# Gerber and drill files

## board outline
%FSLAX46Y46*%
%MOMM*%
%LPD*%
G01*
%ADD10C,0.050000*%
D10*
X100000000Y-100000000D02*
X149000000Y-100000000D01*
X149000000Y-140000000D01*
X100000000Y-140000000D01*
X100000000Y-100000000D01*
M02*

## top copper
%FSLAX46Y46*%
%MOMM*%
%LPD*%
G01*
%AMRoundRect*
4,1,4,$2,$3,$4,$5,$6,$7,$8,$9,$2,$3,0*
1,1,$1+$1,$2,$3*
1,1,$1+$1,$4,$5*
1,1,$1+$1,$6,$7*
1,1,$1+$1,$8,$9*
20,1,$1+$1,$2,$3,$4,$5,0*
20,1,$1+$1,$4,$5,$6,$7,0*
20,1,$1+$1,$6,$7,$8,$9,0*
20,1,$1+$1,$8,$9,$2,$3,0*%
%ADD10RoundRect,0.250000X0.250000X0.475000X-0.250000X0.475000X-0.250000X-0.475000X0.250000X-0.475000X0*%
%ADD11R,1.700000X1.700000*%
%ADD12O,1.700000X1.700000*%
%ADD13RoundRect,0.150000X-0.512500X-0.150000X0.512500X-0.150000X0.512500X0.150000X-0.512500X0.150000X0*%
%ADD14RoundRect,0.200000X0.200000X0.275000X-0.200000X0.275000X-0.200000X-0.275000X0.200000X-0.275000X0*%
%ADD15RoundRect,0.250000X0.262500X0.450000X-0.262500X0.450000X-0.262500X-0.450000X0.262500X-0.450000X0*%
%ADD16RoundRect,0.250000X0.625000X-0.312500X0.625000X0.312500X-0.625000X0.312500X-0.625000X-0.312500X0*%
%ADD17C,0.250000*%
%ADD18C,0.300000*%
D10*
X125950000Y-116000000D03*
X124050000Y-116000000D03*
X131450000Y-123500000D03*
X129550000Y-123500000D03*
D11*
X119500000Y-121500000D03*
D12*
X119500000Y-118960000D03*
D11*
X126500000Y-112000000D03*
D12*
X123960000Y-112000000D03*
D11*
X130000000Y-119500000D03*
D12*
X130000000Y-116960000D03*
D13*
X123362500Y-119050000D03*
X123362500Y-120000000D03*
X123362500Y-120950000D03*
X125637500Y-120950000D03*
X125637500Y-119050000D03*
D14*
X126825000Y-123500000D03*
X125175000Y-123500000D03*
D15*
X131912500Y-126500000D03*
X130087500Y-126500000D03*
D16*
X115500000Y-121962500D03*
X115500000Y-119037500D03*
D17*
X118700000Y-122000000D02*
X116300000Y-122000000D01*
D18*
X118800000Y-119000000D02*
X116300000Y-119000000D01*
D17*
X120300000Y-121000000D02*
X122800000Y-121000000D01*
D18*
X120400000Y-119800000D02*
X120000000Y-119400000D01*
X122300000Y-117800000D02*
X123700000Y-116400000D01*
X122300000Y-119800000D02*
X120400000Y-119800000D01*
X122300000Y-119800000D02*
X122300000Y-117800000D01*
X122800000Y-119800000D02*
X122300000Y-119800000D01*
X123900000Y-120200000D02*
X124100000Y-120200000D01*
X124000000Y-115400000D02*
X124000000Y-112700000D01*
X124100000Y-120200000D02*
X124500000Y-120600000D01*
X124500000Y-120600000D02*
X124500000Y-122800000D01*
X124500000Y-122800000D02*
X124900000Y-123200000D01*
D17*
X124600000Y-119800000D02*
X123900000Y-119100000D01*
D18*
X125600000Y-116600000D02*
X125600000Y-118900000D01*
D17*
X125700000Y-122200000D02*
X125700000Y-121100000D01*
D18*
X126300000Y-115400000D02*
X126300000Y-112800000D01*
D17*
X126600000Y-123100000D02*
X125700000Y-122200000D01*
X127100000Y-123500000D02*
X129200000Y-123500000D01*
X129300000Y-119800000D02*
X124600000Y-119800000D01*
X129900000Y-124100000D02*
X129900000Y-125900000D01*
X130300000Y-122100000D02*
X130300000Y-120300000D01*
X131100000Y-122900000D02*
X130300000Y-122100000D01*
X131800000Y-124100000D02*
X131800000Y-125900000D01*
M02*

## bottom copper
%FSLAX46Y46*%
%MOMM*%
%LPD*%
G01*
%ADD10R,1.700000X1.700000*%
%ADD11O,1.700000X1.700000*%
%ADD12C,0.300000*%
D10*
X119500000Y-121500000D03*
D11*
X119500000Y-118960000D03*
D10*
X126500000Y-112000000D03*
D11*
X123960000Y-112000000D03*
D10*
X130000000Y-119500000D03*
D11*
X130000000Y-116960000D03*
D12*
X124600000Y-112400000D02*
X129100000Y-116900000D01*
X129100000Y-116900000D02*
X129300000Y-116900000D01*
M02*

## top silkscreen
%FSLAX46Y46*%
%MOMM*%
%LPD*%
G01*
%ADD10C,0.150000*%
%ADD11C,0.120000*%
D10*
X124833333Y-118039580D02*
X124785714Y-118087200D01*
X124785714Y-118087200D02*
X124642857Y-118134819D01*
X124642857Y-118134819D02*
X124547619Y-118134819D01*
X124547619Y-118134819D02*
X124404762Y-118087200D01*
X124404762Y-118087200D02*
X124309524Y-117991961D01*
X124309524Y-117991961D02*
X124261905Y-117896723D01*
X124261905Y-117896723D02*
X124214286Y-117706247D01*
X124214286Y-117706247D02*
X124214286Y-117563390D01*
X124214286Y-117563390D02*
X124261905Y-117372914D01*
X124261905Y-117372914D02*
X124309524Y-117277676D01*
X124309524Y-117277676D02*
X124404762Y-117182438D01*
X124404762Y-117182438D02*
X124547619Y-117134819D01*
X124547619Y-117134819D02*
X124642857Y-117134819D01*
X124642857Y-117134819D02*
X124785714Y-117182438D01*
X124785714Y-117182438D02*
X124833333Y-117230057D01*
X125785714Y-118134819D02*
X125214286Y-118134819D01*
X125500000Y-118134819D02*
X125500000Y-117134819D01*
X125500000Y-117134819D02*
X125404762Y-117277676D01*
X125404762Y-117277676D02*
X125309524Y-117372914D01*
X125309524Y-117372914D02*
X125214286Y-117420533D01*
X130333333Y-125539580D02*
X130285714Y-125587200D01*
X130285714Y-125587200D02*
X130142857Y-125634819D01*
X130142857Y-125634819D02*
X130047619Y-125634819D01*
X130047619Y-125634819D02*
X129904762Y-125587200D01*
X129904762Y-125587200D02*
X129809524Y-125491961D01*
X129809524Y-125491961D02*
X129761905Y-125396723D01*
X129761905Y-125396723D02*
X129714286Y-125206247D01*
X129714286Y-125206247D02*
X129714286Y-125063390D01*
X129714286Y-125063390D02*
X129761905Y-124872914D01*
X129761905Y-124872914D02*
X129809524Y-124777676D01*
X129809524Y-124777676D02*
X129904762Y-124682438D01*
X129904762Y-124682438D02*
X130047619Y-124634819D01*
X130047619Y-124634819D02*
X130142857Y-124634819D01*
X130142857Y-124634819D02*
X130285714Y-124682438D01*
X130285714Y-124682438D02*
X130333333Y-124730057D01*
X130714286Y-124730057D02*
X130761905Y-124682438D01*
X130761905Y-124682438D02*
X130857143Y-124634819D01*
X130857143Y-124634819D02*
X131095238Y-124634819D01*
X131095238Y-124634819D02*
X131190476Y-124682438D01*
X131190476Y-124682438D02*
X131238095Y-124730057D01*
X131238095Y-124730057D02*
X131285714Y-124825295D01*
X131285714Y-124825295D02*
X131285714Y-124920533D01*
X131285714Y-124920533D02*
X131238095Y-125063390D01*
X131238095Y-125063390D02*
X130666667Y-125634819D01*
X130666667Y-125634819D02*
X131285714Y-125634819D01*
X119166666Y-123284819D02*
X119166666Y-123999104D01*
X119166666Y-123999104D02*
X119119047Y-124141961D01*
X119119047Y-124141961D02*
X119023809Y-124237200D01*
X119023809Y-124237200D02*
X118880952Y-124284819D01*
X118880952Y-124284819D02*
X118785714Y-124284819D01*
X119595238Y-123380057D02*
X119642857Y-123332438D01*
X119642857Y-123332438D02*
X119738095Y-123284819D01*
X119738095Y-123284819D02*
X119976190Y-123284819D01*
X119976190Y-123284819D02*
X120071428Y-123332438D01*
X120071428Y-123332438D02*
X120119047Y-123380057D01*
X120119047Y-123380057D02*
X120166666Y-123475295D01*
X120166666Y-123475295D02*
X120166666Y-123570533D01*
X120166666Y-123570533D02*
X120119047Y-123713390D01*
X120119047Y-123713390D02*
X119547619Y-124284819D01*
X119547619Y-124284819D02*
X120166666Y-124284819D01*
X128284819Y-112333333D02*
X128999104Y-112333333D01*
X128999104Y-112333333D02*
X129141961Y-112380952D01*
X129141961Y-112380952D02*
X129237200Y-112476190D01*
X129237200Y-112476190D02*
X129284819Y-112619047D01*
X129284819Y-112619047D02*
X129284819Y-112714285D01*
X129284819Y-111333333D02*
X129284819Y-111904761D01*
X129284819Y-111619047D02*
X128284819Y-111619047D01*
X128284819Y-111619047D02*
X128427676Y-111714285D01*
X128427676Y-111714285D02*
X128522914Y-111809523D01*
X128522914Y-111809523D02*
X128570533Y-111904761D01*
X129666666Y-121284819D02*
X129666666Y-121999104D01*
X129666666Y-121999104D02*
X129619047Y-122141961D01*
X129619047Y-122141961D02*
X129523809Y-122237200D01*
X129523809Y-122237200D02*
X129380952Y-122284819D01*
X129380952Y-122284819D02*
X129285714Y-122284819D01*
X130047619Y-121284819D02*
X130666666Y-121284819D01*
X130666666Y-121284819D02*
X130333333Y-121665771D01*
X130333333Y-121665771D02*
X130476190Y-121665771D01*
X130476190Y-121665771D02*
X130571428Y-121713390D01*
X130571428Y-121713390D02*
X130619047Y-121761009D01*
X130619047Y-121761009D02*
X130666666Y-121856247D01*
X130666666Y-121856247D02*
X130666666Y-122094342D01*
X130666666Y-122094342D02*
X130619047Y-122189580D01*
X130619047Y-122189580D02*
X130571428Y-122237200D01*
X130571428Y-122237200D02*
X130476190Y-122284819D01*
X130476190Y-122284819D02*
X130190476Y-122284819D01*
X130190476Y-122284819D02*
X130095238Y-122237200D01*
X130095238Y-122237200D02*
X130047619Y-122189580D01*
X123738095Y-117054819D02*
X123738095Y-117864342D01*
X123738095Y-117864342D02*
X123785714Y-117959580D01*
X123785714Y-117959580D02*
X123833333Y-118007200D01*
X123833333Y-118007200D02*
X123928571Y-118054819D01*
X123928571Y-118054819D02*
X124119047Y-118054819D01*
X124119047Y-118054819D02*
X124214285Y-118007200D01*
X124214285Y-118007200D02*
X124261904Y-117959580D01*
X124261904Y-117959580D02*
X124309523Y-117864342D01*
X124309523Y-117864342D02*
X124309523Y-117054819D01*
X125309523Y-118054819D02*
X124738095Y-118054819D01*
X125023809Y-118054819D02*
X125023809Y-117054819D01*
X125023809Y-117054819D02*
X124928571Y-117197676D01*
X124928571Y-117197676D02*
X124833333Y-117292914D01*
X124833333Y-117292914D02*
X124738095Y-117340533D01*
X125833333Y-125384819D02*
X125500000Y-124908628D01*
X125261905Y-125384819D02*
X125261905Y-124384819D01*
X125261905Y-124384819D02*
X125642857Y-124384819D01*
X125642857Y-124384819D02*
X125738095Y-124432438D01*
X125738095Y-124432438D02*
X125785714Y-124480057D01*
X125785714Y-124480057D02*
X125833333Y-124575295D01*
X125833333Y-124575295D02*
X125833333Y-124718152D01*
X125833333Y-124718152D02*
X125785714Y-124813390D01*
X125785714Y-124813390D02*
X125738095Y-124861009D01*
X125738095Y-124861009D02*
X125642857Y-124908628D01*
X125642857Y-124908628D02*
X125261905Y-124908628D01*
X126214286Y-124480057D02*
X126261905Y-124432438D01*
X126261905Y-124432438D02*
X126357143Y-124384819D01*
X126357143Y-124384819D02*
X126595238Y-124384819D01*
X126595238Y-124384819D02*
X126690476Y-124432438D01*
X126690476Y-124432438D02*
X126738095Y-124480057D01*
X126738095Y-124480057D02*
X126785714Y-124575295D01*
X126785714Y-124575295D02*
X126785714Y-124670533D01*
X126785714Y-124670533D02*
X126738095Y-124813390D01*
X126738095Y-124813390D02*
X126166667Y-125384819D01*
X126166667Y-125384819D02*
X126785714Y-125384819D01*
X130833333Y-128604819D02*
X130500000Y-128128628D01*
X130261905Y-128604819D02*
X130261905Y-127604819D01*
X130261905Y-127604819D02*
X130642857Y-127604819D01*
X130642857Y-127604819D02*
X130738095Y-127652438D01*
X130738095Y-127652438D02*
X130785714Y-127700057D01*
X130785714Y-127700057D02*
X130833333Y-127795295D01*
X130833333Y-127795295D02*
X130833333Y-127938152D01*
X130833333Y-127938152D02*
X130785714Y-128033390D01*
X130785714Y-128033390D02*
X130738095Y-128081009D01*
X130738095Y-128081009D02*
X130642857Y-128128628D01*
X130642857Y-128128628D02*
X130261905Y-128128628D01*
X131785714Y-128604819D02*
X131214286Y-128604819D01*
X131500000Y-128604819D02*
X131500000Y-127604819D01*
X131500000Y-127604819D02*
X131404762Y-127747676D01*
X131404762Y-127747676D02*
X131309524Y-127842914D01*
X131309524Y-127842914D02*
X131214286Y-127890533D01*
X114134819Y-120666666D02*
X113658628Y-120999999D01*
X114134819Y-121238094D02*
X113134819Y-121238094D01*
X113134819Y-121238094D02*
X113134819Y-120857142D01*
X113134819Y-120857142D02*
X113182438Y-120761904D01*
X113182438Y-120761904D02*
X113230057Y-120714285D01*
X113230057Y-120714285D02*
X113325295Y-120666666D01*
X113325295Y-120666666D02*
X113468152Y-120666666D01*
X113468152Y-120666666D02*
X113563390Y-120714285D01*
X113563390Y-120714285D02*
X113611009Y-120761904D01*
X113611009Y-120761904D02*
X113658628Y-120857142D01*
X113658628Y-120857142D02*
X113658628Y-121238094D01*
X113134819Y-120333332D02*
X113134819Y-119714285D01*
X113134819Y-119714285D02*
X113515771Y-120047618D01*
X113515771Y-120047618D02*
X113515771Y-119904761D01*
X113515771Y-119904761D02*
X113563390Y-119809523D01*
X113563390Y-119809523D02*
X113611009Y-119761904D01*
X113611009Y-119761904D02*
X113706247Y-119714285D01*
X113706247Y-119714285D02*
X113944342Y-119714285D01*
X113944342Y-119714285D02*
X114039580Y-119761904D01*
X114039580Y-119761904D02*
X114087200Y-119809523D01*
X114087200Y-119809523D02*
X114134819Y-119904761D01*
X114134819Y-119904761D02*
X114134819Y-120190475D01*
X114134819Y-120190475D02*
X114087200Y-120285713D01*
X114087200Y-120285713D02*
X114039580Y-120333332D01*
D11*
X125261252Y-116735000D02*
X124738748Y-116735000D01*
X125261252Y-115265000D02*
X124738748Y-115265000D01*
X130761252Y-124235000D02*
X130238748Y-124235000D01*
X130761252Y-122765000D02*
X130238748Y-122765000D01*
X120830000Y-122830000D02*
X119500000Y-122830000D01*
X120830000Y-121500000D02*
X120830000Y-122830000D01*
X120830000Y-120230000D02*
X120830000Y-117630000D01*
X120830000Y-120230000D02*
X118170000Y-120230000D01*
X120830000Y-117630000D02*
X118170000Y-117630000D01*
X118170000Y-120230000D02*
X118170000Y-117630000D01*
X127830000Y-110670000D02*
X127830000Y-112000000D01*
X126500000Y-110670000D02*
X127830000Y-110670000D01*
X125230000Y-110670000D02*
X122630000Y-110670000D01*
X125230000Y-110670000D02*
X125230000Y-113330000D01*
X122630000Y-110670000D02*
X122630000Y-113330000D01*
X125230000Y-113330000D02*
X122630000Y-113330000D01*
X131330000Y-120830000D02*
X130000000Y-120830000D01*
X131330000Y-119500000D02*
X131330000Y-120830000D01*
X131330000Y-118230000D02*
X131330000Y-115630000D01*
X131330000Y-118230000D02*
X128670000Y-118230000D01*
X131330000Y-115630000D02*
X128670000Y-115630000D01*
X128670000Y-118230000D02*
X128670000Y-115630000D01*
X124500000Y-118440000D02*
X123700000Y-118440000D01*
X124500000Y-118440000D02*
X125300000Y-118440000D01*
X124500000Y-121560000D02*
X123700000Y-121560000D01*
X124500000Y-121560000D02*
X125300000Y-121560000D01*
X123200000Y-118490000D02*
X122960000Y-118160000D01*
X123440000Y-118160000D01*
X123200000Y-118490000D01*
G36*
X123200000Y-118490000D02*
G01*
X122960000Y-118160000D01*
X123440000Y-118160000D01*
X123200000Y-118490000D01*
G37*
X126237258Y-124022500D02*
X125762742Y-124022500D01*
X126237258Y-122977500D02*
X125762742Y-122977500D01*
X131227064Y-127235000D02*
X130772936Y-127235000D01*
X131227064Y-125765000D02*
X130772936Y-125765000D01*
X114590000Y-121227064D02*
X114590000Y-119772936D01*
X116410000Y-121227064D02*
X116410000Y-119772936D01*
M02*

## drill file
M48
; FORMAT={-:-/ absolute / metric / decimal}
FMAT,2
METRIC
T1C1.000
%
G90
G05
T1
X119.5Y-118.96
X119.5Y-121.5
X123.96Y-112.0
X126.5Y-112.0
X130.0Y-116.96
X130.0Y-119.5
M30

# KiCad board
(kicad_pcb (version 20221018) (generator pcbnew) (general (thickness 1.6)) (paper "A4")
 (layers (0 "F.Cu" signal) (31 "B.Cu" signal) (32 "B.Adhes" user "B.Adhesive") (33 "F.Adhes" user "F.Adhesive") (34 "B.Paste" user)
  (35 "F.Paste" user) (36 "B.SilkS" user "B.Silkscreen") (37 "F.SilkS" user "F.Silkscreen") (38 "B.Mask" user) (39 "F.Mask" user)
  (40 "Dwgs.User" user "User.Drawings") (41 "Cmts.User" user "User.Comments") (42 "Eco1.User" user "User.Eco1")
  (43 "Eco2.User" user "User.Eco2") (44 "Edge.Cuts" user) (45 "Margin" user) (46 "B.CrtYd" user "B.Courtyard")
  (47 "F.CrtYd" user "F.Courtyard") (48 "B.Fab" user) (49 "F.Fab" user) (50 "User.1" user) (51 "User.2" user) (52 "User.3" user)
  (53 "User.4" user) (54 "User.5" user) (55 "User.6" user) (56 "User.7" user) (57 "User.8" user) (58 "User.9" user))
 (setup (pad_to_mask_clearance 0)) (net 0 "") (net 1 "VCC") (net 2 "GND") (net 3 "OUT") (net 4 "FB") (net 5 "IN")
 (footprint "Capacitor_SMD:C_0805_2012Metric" (layer "F.Cu") (at 125 116 180)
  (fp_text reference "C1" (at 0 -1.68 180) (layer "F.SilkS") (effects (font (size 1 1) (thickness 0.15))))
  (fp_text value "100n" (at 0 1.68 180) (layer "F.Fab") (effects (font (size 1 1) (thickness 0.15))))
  (fp_line (start -0.261252 -0.735) (end 0.261252 -0.735) (stroke (width 0.12) (type solid)) (layer "F.SilkS"))
  (fp_line (start -0.261252 0.735) (end 0.261252 0.735) (stroke (width 0.12) (type solid)) (layer "F.SilkS"))
  (pad "1" smd roundrect (at -0.95 0 180) (size 1 1.45) (layers "F.Cu" "F.Paste" "F.Mask") (roundrect_rratio 0.25) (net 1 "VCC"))
  (pad "2" smd roundrect (at 0.95 0 180) (size 1 1.45) (layers "F.Cu" "F.Paste" "F.Mask") (roundrect_rratio 0.25) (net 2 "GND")))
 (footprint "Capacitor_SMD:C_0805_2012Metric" (layer "F.Cu") (at 130.5 123.5 180)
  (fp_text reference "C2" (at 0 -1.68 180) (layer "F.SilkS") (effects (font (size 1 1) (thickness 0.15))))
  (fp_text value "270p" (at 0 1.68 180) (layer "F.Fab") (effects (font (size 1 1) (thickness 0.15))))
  (fp_line (start -0.261252 -0.735) (end 0.261252 -0.735) (stroke (width 0.12) (type solid)) (layer "F.SilkS"))
  (fp_line (start -0.261252 0.735) (end 0.261252 0.735) (stroke (width 0.12) (type solid)) (layer "F.SilkS"))
  (pad "1" smd roundrect (at -0.95 0 180) (size 1 1.45) (layers "F.Cu" "F.Paste" "F.Mask") (roundrect_rratio 0.25) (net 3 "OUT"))
  (pad "2" smd roundrect (at 0.95 0 180) (size 1 1.45) (layers "F.Cu" "F.Paste" "F.Mask") (roundrect_rratio 0.25) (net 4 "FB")))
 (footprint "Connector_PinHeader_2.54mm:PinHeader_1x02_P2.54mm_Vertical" (layer "F.Cu") (at 119.5 121.5 180)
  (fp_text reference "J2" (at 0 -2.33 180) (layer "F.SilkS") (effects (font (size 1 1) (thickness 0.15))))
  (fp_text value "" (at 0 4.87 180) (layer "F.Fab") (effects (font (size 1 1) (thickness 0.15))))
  (fp_line (start -1.33 -1.33) (end 0 -1.33) (stroke (width 0.12) (type solid)) (layer "F.SilkS"))
  (fp_line (start -1.33 0) (end -1.33 -1.33) (stroke (width 0.12) (type solid)) (layer "F.SilkS"))
  (fp_line (start -1.33 1.27) (end -1.33 3.87) (stroke (width 0.12) (type solid)) (layer "F.SilkS"))
  (fp_line (start -1.33 1.27) (end 1.33 1.27) (stroke (width 0.12) (type solid)) (layer "F.SilkS"))
  (fp_line (start -1.33 3.87) (end 1.33 3.87) (stroke (width 0.12) (type solid)) (layer "F.SilkS"))
  (fp_line (start 1.33 1.27) (end 1.33 3.87) (stroke (width 0.12) (type solid)) (layer "F.SilkS"))
  (pad "1" thru_hole rect (at 0 0 180) (size 1.7 1.7) (drill 1) (layers "*.Cu" "*.Mask") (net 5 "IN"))
  (pad "2" thru_hole oval (at 0 2.54 180) (size 1.7 1.7) (drill 1) (layers "*.Cu" "*.Mask") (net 2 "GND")))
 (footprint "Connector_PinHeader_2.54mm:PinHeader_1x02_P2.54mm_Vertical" (layer "F.Cu") (at 126.5 112 -90)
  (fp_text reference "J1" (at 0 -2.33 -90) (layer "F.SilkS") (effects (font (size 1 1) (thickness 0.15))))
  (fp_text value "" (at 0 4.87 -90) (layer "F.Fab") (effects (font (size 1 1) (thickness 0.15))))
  (fp_line (start -1.33 -1.33) (end 0 -1.33) (stroke (width 0.12) (type solid)) (layer "F.SilkS"))
  (fp_line (start -1.33 0) (end -1.33 -1.33) (stroke (width 0.12) (type solid)) (layer "F.SilkS"))
  (fp_line (start -1.33 1.27) (end -1.33 3.87) (stroke (width 0.12) (type solid)) (layer "F.SilkS"))
  (fp_line (start -1.33 1.27) (end 1.33 1.27) (stroke (width 0.12) (type solid)) (layer "F.SilkS"))
  (fp_line (start -1.33 3.87) (end 1.33 3.87) (stroke (width 0.12) (type solid)) (layer "F.SilkS"))
  (fp_line (start 1.33 1.27) (end 1.33 3.87) (stroke (width 0.12) (type solid)) (layer "F.SilkS"))
  (pad "1" thru_hole rect (at 0 0 270) (size 1.7 1.7) (drill 1) (layers "*.Cu" "*.Mask") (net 1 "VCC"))
  (pad "2" thru_hole oval (at 0 2.54 270) (size 1.7 1.7) (drill 1) (layers "*.Cu" "*.Mask") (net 2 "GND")))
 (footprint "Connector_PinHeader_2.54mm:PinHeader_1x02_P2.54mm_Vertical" (layer "F.Cu") (at 130 119.5 180)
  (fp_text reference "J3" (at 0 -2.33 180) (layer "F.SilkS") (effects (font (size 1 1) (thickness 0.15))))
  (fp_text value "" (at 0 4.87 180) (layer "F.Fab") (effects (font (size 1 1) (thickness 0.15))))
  (fp_line (start -1.33 -1.33) (end 0 -1.33) (stroke (width 0.12) (type solid)) (layer "F.SilkS"))
  (fp_line (start -1.33 0) (end -1.33 -1.33) (stroke (width 0.12) (type solid)) (layer "F.SilkS"))
  (fp_line (start -1.33 1.27) (end -1.33 3.87) (stroke (width 0.12) (type solid)) (layer "F.SilkS"))
  (fp_line (start -1.33 1.27) (end 1.33 1.27) (stroke (width 0.12) (type solid)) (layer "F.SilkS"))
  (fp_line (start -1.33 3.87) (end 1.33 3.87) (stroke (width 0.12) (type solid)) (layer "F.SilkS"))
  (fp_line (start 1.33 1.27) (end 1.33 3.87) (stroke (width 0.12) (type solid)) (layer "F.SilkS"))
  (pad "1" thru_hole rect (at 0 0 180) (size 1.7 1.7) (drill 1) (layers "*.Cu" "*.Mask") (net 3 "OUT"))
  (pad "2" thru_hole oval (at 0 2.54 180) (size 1.7 1.7) (drill 1) (layers "*.Cu" "*.Mask") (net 2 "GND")))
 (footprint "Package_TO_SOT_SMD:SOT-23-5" (layer "F.Cu") (at 124.5 120)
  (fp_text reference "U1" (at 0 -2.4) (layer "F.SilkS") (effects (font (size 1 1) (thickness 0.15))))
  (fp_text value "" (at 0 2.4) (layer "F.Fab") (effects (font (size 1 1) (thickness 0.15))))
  (fp_line (start 0 -1.56) (end -0.8 -1.56) (stroke (width 0.12) (type solid)) (layer "F.SilkS"))
  (fp_line (start 0 -1.56) (end 0.8 -1.56) (stroke (width 0.12) (type solid)) (layer "F.SilkS"))
  (fp_line (start 0 1.56) (end -0.8 1.56) (stroke (width 0.12) (type solid)) (layer "F.SilkS"))
  (fp_line (start 0 1.56) (end 0.8 1.56) (stroke (width 0.12) (type solid)) (layer "F.SilkS"))
  (fp_poly
   (pts (xy -1.3 -1.51) (xy -1.54 -1.84) (xy -1.06 -1.84) (xy -1.3 -1.51)) (stroke (width 0.12) (type solid)) (fill solid) (layer "F.SilkS"))
  (pad "1" smd roundrect (at -1.1375 -0.95) (size 1.325 0.6) (layers "F.Cu" "F.Paste" "F.Mask") (roundrect_rratio 0.25) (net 3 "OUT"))
  (pad "2" smd roundrect (at -1.1375 0) (size 1.325 0.6) (layers "F.Cu" "F.Paste" "F.Mask") (roundrect_rratio 0.25) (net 2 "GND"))
  (pad "3" smd roundrect (at -1.1375 0.95) (size 1.325 0.6) (layers "F.Cu" "F.Paste" "F.Mask") (roundrect_rratio 0.25) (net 5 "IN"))
  (pad "4" smd roundrect (at 1.1375 0.95) (size 1.325 0.6) (layers "F.Cu" "F.Paste" "F.Mask") (roundrect_rratio 0.25) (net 4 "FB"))
  (pad "5" smd roundrect (at 1.1375 -0.95) (size 1.325 0.6) (layers "F.Cu" "F.Paste" "F.Mask") (roundrect_rratio 0.25) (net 1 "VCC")))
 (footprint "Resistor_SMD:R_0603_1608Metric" (layer "F.Cu") (at 126 123.5 180)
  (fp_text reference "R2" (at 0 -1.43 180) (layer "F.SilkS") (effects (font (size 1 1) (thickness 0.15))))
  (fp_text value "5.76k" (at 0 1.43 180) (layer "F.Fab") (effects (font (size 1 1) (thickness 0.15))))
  (fp_line (start -0.237258 -0.5225) (end 0.237258 -0.5225) (stroke (width 0.12) (type solid)) (layer "F.SilkS"))
  (fp_line (start -0.237258 0.5225) (end 0.237258 0.5225) (stroke (width 0.12) (type solid)) (layer "F.SilkS"))
  (pad "1" smd roundrect (at -0.825 0 180) (size 0.8 0.95) (layers "F.Cu" "F.Paste" "F.Mask") (roundrect_rratio 0.25) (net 4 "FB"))
  (pad "2" smd roundrect (at 0.825 0 180) (size 0.8 0.95) (layers "F.Cu" "F.Paste" "F.Mask") (roundrect_rratio 0.25) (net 2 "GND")))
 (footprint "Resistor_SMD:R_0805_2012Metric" (layer "F.Cu") (at 131 126.5 180)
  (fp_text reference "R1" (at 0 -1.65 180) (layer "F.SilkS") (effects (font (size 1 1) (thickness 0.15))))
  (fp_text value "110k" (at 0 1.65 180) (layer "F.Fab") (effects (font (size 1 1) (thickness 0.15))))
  (fp_line (start -0.227064 -0.735) (end 0.227064 -0.735) (stroke (width 0.12) (type solid)) (layer "F.SilkS"))
  (fp_line (start -0.227064 0.735) (end 0.227064 0.735) (stroke (width 0.12) (type solid)) (layer "F.SilkS"))
  (pad "1" smd roundrect (at -0.9125 0 180) (size 1.025 1.4) (layers "F.Cu" "F.Paste" "F.Mask") (roundrect_rratio 0.243902) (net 3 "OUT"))
  (pad "2" smd roundrect (at 0.9125 0 180) (size 1.025 1.4) (layers "F.Cu" "F.Paste" "F.Mask") (roundrect_rratio 0.243902) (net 4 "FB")))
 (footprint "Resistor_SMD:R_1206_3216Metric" (layer "F.Cu") (at 115.5 120.5 90)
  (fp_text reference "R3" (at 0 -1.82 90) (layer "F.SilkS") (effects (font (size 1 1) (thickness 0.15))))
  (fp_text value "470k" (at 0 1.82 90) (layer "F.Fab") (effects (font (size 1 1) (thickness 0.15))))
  (fp_line (start -0.727064 -0.91) (end 0.727064 -0.91) (stroke (width 0.12) (type solid)) (layer "F.SilkS"))
  (fp_line (start -0.727064 0.91) (end 0.727064 0.91) (stroke (width 0.12) (type solid)) (layer "F.SilkS"))
  (pad "1" smd roundrect (at -1.4625 0 90) (size 1.125 1.75) (layers "F.Cu" "F.Paste" "F.Mask") (roundrect_rratio 0.222222) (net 5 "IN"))
  (pad "2" smd roundrect (at 1.4625 0 90) (size 1.125 1.75) (layers "F.Cu" "F.Paste" "F.Mask") (roundrect_rratio 0.222222) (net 2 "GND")))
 (gr_rect (start 100 100) (end 149 140) (stroke (width 0.05) (type default)) (fill none) (layer "Edge.Cuts"))
 (segment (start 118.7 122) (end 116.3 122) (width 0.25) (layer "F.Cu") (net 5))
 (segment (start 118.8 119) (end 116.3 119) (width 0.3) (layer "F.Cu") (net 2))
 (segment (start 120.3 121) (end 122.8 121) (width 0.25) (layer "F.Cu") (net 5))
 (segment (start 120.4 119.8) (end 120 119.4) (width 0.3) (layer "F.Cu") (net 2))
 (segment (start 122.3 117.8) (end 123.7 116.4) (width 0.3) (layer "F.Cu") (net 2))
 (segment (start 122.3 119.8) (end 120.4 119.8) (width 0.3) (layer "F.Cu") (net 2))
 (segment (start 122.3 119.8) (end 122.3 117.8) (width 0.3) (layer "F.Cu") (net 2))
 (segment (start 122.8 119.8) (end 122.3 119.8) (width 0.3) (layer "F.Cu") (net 2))
 (segment (start 123.9 120.2) (end 124.1 120.2) (width 0.3) (layer "F.Cu") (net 2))
 (segment (start 124 115.4) (end 124 112.7) (width 0.3) (layer "F.Cu") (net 2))
 (segment (start 124.1 120.2) (end 124.5 120.6) (width 0.3) (layer "F.Cu") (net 2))
 (segment (start 124.5 120.6) (end 124.5 122.8) (width 0.3) (layer "F.Cu") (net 2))
 (segment (start 124.5 122.8) (end 124.9 123.2) (width 0.3) (layer "F.Cu") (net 2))
 (segment (start 124.6 112.4) (end 129.1 116.9) (width 0.3) (layer "B.Cu") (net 2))
 (segment (start 124.6 119.8) (end 123.9 119.1) (width 0.25) (layer "F.Cu") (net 3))
 (segment (start 125.6 116.6) (end 125.6 118.9) (width 0.3) (layer "F.Cu") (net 1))
 (segment (start 125.7 122.2) (end 125.7 121.1) (width 0.25) (layer "F.Cu") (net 4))
 (segment (start 126.3 115.4) (end 126.3 112.8) (width 0.3) (layer "F.Cu") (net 1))
 (segment (start 126.6 123.1) (end 125.7 122.2) (width 0.25) (layer "F.Cu") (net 4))
 (segment (start 127.1 123.5) (end 129.2 123.5) (width 0.25) (layer "F.Cu") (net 4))
 (segment (start 129.1 116.9) (end 129.3 116.9) (width 0.3) (layer "B.Cu") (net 2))
 (segment (start 129.3 119.8) (end 124.6 119.8) (width 0.25) (layer "F.Cu") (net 3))
 (segment (start 129.9 124.1) (end 129.9 125.9) (width 0.25) (layer "F.Cu") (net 4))
 (segment (start 130.3 122.1) (end 130.3 120.3) (width 0.25) (layer "F.Cu") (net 3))
 (segment (start 131.1 122.9) (end 130.3 122.1) (width 0.25) (layer "F.Cu") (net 3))
 (segment (start 131.8 124.1) (end 131.8 125.9) (width 0.25) (layer "F.Cu") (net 3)))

